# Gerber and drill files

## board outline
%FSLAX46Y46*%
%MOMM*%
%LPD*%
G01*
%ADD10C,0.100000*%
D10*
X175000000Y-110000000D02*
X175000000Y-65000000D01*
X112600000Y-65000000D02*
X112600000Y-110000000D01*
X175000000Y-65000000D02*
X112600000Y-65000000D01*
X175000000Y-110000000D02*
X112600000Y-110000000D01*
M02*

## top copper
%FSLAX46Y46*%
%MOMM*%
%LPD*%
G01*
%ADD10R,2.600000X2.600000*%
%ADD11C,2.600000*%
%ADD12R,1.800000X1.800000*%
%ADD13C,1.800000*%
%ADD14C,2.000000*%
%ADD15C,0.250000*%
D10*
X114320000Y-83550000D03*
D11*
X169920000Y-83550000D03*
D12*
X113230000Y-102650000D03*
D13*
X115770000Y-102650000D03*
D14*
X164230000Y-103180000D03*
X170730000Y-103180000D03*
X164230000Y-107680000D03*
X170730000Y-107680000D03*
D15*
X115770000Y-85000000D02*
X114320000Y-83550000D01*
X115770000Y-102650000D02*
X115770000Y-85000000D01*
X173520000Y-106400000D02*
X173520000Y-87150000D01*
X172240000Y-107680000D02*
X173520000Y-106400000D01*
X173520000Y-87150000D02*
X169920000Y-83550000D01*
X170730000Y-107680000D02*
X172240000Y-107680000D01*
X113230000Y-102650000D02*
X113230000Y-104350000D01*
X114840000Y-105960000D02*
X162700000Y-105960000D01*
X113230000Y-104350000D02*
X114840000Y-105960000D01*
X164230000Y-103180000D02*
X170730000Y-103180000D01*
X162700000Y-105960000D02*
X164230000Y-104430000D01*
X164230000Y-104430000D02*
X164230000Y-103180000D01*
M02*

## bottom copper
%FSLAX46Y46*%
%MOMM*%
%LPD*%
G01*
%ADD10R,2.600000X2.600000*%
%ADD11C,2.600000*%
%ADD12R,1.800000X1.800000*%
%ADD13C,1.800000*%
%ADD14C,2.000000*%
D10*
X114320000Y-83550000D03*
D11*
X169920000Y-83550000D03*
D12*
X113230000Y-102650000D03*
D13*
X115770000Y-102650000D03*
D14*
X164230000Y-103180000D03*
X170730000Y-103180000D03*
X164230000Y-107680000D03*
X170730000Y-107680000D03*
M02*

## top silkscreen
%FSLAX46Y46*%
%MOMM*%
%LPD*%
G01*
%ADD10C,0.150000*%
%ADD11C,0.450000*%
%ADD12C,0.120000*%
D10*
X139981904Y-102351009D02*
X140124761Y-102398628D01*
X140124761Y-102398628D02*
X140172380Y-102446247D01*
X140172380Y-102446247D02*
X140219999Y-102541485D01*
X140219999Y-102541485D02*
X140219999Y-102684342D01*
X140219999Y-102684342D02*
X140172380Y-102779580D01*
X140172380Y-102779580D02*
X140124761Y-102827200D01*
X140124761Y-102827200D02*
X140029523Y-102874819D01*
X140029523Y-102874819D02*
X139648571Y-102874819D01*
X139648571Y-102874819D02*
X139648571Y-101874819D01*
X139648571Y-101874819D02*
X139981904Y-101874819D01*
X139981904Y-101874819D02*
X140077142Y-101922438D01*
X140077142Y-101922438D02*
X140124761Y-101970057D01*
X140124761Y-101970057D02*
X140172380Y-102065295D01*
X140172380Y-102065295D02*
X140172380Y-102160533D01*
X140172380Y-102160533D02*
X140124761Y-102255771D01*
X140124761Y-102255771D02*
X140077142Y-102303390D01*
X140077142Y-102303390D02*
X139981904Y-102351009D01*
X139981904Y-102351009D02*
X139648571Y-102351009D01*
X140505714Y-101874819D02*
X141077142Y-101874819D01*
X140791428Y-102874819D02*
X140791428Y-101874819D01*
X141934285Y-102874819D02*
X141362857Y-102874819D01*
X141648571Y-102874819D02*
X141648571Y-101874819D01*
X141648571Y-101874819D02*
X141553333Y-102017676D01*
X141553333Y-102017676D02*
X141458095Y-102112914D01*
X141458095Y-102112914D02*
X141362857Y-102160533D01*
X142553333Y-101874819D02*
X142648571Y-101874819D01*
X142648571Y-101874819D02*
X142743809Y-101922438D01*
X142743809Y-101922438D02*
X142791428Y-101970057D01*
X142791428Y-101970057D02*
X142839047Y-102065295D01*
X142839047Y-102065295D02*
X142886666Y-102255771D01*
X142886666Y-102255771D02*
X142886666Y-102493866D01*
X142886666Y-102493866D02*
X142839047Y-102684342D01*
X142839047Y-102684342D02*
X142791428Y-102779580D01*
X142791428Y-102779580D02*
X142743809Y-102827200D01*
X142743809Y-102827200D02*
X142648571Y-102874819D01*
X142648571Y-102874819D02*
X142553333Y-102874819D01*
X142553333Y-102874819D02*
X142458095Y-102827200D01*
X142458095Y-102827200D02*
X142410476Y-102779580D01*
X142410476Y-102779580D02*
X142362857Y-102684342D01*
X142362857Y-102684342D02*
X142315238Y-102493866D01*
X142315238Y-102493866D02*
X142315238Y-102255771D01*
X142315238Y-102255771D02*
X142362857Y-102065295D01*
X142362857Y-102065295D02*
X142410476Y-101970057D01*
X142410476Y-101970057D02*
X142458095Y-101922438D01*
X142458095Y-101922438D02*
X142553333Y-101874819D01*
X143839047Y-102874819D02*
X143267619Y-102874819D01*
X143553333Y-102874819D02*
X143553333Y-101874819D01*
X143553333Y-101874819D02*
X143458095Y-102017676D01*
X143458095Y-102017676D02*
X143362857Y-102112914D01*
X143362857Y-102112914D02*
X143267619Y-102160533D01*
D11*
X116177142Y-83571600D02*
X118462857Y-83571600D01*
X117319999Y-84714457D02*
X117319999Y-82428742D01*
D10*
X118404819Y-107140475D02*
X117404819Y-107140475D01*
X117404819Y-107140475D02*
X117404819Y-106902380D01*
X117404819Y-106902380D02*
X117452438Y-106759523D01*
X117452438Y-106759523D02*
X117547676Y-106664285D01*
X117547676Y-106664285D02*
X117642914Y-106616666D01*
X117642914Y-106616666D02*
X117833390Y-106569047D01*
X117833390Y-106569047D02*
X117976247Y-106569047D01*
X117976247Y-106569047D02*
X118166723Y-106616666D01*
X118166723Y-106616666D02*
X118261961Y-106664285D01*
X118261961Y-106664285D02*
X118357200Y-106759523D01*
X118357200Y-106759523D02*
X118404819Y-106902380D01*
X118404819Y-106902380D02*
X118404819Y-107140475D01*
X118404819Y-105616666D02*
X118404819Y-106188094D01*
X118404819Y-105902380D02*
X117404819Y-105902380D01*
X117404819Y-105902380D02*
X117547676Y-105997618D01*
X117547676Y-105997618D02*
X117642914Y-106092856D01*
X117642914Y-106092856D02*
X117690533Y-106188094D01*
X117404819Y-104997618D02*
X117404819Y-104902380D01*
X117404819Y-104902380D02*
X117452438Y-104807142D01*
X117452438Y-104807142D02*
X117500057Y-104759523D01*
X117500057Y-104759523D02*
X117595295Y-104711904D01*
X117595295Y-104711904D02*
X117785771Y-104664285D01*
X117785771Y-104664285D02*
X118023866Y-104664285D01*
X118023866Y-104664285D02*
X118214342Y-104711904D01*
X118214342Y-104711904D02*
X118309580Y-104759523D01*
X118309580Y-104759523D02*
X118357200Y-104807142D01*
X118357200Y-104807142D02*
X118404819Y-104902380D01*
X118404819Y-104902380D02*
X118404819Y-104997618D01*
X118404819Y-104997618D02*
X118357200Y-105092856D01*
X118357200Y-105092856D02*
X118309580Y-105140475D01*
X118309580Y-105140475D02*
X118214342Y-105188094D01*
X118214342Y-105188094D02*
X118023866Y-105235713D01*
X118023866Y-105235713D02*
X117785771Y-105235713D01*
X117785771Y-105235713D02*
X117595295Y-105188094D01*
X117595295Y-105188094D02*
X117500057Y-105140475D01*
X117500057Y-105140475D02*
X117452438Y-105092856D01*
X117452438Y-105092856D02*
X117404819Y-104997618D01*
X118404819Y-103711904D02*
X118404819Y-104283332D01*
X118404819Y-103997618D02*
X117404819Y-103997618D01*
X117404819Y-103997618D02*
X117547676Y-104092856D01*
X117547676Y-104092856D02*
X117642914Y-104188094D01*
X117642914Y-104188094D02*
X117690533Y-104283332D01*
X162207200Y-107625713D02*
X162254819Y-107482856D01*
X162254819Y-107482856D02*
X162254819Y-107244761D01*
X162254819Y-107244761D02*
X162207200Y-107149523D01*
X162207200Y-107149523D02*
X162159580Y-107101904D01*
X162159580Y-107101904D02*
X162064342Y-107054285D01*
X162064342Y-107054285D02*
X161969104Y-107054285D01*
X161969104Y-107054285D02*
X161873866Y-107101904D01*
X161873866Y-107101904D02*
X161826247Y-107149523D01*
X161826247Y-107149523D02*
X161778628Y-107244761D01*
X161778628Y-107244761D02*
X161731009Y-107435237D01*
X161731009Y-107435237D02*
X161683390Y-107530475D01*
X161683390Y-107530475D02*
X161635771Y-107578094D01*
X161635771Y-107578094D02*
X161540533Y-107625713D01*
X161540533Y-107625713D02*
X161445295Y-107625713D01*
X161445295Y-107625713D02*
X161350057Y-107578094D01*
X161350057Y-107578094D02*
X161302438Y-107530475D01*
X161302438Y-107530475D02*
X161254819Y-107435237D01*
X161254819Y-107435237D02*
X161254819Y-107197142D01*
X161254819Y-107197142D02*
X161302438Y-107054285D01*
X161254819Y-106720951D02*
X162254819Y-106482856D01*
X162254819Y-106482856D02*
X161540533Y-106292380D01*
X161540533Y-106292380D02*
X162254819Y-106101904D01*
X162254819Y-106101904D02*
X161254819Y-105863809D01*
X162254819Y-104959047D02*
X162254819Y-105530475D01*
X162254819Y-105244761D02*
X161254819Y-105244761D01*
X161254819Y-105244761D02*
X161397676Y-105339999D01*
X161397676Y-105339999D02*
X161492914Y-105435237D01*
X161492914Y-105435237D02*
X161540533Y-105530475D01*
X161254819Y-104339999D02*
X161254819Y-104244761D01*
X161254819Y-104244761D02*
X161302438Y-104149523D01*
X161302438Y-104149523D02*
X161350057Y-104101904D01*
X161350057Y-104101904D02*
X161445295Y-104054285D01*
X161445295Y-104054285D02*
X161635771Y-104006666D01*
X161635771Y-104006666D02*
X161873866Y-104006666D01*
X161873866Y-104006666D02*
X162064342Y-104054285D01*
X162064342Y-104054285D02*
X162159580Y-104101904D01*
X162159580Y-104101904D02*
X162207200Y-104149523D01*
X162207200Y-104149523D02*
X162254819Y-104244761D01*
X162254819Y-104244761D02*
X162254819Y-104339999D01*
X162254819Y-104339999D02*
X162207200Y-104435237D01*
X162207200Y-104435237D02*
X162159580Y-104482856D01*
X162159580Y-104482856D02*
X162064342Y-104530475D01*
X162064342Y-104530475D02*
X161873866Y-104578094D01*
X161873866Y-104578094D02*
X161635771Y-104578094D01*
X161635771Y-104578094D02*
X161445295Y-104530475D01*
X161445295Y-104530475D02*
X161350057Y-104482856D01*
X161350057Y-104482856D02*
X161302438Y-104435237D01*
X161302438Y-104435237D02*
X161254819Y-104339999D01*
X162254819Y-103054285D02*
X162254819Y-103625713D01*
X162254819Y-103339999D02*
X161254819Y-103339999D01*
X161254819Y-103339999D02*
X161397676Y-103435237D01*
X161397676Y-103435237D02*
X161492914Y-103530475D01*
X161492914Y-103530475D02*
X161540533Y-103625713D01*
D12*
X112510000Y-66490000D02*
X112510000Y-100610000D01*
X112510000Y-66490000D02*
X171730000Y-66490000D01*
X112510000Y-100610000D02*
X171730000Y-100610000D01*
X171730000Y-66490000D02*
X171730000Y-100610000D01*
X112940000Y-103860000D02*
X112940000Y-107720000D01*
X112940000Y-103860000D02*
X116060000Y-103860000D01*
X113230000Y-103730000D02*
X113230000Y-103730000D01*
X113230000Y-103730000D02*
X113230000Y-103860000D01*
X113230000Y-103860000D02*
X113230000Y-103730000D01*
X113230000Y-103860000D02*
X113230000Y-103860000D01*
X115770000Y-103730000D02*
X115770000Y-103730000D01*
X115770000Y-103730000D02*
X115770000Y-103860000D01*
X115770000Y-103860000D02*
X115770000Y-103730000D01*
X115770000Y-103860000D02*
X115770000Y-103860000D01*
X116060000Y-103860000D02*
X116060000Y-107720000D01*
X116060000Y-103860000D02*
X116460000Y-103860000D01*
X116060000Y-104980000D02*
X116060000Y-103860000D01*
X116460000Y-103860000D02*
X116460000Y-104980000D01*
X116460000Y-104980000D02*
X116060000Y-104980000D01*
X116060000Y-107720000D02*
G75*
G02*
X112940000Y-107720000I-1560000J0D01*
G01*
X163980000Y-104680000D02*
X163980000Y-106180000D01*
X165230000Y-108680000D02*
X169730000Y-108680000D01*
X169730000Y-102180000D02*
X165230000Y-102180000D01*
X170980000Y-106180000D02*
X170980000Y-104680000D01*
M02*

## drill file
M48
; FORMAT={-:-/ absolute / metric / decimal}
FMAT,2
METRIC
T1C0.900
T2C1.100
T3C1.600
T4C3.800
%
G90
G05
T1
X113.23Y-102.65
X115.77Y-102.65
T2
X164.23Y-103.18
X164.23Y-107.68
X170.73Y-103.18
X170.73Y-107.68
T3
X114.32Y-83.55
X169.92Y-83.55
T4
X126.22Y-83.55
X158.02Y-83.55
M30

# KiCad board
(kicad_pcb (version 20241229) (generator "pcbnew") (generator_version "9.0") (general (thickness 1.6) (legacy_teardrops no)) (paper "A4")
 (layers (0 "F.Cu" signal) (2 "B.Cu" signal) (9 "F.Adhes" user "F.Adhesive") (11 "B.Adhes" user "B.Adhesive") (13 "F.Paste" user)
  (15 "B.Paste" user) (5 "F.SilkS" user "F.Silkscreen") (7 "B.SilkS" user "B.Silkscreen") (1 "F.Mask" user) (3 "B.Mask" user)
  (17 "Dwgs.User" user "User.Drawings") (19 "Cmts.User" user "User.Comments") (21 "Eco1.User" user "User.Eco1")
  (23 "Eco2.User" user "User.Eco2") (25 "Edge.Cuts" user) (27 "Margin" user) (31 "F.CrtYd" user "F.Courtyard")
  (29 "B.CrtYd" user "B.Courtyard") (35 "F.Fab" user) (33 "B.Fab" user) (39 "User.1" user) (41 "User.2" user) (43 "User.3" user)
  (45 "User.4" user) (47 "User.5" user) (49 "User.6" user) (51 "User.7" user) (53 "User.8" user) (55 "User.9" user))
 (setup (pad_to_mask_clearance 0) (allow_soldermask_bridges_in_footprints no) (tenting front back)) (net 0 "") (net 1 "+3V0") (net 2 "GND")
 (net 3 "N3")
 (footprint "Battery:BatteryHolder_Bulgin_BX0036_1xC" (layer "F.Cu") (at 114.32 83.55)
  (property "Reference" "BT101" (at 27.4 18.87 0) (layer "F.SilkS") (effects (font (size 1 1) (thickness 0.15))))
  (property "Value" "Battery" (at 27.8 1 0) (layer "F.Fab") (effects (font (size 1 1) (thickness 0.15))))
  (fp_line (start -1.81 -17.06) (end -1.81 17.06) (stroke (width 0.12) (type solid)) (layer "F.SilkS"))
  (fp_line (start -1.81 -17.06) (end 57.41 -17.06) (stroke (width 0.12) (type solid)) (layer "F.SilkS"))
  (fp_line (start -1.81 17.06) (end 57.41 17.06) (stroke (width 0.12) (type solid)) (layer "F.SilkS"))
  (fp_line (start 57.41 -17.06) (end 57.41 17.06) (stroke (width 0.12) (type solid)) (layer "F.SilkS"))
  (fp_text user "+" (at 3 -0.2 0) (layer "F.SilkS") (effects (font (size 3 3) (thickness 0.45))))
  (pad "" np_thru_hole circle (at 11.9 0) (size 3.8 3.8) (drill 3.8) (layers "*.Cu" "*.Mask"))
  (pad "" np_thru_hole circle (at 43.7 0) (size 3.8 3.8) (drill 3.8) (layers "*.Cu" "*.Mask"))
  (pad "1" thru_hole rect (at 0 0) (size 2.6 2.6) (drill 1.6) (layers "*.Cu" "*.Mask") (remove_unused_layers no) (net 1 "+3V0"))
  (pad "2" thru_hole circle (at 55.6 0) (size 2.6 2.6) (drill 1.6) (layers "*.Cu" "*.Mask") (remove_unused_layers no) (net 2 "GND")))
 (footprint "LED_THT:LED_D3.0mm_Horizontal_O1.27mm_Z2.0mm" (layer "F.Cu") (at 113.23 102.65)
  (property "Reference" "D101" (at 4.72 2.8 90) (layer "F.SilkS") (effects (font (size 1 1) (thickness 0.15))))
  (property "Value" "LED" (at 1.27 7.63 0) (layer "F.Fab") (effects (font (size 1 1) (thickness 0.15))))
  (fp_line (start -0.29 1.21) (end -0.29 5.07) (stroke (width 0.12) (type solid)) (layer "F.SilkS"))
  (fp_line (start -0.29 1.21) (end 2.83 1.21) (stroke (width 0.12) (type solid)) (layer "F.SilkS"))
  (fp_line (start 0 1.08) (end 0 1.08) (stroke (width 0.12) (type solid)) (layer "F.SilkS"))
  (fp_line (start 0 1.08) (end 0 1.21) (stroke (width 0.12) (type solid)) (layer "F.SilkS"))
  (fp_line (start 0 1.21) (end 0 1.08) (stroke (width 0.12) (type solid)) (layer "F.SilkS"))
  (fp_line (start 0 1.21) (end 0 1.21) (stroke (width 0.12) (type solid)) (layer "F.SilkS"))
  (fp_line (start 2.54 1.08) (end 2.54 1.08) (stroke (width 0.12) (type solid)) (layer "F.SilkS"))
  (fp_line (start 2.54 1.08) (end 2.54 1.21) (stroke (width 0.12) (type solid)) (layer "F.SilkS"))
  (fp_line (start 2.54 1.21) (end 2.54 1.08) (stroke (width 0.12) (type solid)) (layer "F.SilkS"))
  (fp_line (start 2.54 1.21) (end 2.54 1.21) (stroke (width 0.12) (type solid)) (layer "F.SilkS"))
  (fp_line (start 2.83 1.21) (end 2.83 5.07) (stroke (width 0.12) (type solid)) (layer "F.SilkS"))
  (fp_line (start 2.83 1.21) (end 3.23 1.21) (stroke (width 0.12) (type solid)) (layer "F.SilkS"))
  (fp_line (start 2.83 2.33) (end 2.83 1.21) (stroke (width 0.12) (type solid)) (layer "F.SilkS"))
  (fp_line (start 3.23 1.21) (end 3.23 2.33) (stroke (width 0.12) (type solid)) (layer "F.SilkS"))
  (fp_line (start 3.23 2.33) (end 2.83 2.33) (stroke (width 0.12) (type solid)) (layer "F.SilkS"))
  (fp_arc (start 2.83 5.07) (mid 1.27 6.63) (end -0.29 5.07) (stroke (width 0.12) (type solid)) (layer "F.SilkS"))
  (pad "1" thru_hole rect (at 0 0) (size 1.8 1.8) (drill 0.9) (layers "*.Cu" "*.Mask") (remove_unused_layers no) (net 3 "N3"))
  (pad "2" thru_hole circle (at 2.54 0) (size 1.8 1.8) (drill 0.9) (layers "*.Cu" "*.Mask") (remove_unused_layers no) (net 1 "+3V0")))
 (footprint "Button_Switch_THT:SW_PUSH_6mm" (layer "F.Cu") (at 164.23 103.18)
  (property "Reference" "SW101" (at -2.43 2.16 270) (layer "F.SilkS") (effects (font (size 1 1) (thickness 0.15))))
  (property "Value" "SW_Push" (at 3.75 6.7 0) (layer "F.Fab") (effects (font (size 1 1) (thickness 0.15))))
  (fp_line (start -0.25 1.5) (end -0.25 3) (stroke (width 0.12) (type solid)) (layer "F.SilkS"))
  (fp_line (start 1 5.5) (end 5.5 5.5) (stroke (width 0.12) (type solid)) (layer "F.SilkS"))
  (fp_line (start 5.5 -1) (end 1 -1) (stroke (width 0.12) (type solid)) (layer "F.SilkS"))
  (fp_line (start 6.75 3) (end 6.75 1.5) (stroke (width 0.12) (type solid)) (layer "F.SilkS"))
  (pad "1" thru_hole circle (at 0 0 90) (size 2 2) (drill 1.1) (layers "*.Cu" "*.Mask") (remove_unused_layers no) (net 3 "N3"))
  (pad "1" thru_hole circle (at 6.5 0 90) (size 2 2) (drill 1.1) (layers "*.Cu" "*.Mask") (remove_unused_layers no) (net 3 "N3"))
  (pad "2" thru_hole circle (at 0 4.5 90) (size 2 2) (drill 1.1) (layers "*.Cu" "*.Mask") (remove_unused_layers no) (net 2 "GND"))
  (pad "2" thru_hole circle (at 6.5 4.5 90) (size 2 2) (drill 1.1) (layers "*.Cu" "*.Mask") (remove_unused_layers no) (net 2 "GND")))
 (gr_line (start 175 110) (end 175 65) (stroke (width 0.1) (type default)) (layer "Edge.Cuts"))
 (gr_line (start 112.6 65) (end 112.6 110) (stroke (width 0.1) (type default)) (layer "Edge.Cuts"))
 (gr_line (start 175 65) (end 112.6 65) (stroke (width 0.1) (type default)) (layer "Edge.Cuts"))
 (gr_line (start 175 110) (end 112.6 110) (stroke (width 0.1) (type default)) (layer "Edge.Cuts"))
 (segment (start 115.77 85) (end 114.32 83.55) (width 0.25) (layer "F.Cu") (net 1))
 (segment (start 115.77 102.65) (end 115.77 85) (width 0.25) (layer "F.Cu") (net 1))
 (segment (start 173.52 106.4) (end 173.52 87.15) (width 0.25) (layer "F.Cu") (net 2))
 (segment (start 172.24 107.68) (end 173.52 106.4) (width 0.25) (layer "F.Cu") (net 2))
 (segment (start 173.52 87.15) (end 169.92 83.55) (width 0.25) (layer "F.Cu") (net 2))
 (segment (start 170.73 107.68) (end 172.24 107.68) (width 0.25) (layer "F.Cu") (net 2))
 (segment (start 113.23 102.65) (end 113.23 104.35) (width 0.25) (layer "F.Cu") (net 3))
 (segment (start 114.84 105.96) (end 162.7 105.96) (width 0.25) (layer "F.Cu") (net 3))
 (segment (start 113.23 104.35) (end 114.84 105.96) (width 0.25) (layer "F.Cu") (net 3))
 (segment (start 164.23 103.18) (end 170.73 103.18) (width 0.25) (layer "F.Cu") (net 3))
 (segment (start 162.7 105.96) (end 164.23 104.43) (width 0.25) (layer "F.Cu") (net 3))
 (segment (start 164.23 104.43) (end 164.23 103.18) (width 0.25) (layer "F.Cu") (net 3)))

